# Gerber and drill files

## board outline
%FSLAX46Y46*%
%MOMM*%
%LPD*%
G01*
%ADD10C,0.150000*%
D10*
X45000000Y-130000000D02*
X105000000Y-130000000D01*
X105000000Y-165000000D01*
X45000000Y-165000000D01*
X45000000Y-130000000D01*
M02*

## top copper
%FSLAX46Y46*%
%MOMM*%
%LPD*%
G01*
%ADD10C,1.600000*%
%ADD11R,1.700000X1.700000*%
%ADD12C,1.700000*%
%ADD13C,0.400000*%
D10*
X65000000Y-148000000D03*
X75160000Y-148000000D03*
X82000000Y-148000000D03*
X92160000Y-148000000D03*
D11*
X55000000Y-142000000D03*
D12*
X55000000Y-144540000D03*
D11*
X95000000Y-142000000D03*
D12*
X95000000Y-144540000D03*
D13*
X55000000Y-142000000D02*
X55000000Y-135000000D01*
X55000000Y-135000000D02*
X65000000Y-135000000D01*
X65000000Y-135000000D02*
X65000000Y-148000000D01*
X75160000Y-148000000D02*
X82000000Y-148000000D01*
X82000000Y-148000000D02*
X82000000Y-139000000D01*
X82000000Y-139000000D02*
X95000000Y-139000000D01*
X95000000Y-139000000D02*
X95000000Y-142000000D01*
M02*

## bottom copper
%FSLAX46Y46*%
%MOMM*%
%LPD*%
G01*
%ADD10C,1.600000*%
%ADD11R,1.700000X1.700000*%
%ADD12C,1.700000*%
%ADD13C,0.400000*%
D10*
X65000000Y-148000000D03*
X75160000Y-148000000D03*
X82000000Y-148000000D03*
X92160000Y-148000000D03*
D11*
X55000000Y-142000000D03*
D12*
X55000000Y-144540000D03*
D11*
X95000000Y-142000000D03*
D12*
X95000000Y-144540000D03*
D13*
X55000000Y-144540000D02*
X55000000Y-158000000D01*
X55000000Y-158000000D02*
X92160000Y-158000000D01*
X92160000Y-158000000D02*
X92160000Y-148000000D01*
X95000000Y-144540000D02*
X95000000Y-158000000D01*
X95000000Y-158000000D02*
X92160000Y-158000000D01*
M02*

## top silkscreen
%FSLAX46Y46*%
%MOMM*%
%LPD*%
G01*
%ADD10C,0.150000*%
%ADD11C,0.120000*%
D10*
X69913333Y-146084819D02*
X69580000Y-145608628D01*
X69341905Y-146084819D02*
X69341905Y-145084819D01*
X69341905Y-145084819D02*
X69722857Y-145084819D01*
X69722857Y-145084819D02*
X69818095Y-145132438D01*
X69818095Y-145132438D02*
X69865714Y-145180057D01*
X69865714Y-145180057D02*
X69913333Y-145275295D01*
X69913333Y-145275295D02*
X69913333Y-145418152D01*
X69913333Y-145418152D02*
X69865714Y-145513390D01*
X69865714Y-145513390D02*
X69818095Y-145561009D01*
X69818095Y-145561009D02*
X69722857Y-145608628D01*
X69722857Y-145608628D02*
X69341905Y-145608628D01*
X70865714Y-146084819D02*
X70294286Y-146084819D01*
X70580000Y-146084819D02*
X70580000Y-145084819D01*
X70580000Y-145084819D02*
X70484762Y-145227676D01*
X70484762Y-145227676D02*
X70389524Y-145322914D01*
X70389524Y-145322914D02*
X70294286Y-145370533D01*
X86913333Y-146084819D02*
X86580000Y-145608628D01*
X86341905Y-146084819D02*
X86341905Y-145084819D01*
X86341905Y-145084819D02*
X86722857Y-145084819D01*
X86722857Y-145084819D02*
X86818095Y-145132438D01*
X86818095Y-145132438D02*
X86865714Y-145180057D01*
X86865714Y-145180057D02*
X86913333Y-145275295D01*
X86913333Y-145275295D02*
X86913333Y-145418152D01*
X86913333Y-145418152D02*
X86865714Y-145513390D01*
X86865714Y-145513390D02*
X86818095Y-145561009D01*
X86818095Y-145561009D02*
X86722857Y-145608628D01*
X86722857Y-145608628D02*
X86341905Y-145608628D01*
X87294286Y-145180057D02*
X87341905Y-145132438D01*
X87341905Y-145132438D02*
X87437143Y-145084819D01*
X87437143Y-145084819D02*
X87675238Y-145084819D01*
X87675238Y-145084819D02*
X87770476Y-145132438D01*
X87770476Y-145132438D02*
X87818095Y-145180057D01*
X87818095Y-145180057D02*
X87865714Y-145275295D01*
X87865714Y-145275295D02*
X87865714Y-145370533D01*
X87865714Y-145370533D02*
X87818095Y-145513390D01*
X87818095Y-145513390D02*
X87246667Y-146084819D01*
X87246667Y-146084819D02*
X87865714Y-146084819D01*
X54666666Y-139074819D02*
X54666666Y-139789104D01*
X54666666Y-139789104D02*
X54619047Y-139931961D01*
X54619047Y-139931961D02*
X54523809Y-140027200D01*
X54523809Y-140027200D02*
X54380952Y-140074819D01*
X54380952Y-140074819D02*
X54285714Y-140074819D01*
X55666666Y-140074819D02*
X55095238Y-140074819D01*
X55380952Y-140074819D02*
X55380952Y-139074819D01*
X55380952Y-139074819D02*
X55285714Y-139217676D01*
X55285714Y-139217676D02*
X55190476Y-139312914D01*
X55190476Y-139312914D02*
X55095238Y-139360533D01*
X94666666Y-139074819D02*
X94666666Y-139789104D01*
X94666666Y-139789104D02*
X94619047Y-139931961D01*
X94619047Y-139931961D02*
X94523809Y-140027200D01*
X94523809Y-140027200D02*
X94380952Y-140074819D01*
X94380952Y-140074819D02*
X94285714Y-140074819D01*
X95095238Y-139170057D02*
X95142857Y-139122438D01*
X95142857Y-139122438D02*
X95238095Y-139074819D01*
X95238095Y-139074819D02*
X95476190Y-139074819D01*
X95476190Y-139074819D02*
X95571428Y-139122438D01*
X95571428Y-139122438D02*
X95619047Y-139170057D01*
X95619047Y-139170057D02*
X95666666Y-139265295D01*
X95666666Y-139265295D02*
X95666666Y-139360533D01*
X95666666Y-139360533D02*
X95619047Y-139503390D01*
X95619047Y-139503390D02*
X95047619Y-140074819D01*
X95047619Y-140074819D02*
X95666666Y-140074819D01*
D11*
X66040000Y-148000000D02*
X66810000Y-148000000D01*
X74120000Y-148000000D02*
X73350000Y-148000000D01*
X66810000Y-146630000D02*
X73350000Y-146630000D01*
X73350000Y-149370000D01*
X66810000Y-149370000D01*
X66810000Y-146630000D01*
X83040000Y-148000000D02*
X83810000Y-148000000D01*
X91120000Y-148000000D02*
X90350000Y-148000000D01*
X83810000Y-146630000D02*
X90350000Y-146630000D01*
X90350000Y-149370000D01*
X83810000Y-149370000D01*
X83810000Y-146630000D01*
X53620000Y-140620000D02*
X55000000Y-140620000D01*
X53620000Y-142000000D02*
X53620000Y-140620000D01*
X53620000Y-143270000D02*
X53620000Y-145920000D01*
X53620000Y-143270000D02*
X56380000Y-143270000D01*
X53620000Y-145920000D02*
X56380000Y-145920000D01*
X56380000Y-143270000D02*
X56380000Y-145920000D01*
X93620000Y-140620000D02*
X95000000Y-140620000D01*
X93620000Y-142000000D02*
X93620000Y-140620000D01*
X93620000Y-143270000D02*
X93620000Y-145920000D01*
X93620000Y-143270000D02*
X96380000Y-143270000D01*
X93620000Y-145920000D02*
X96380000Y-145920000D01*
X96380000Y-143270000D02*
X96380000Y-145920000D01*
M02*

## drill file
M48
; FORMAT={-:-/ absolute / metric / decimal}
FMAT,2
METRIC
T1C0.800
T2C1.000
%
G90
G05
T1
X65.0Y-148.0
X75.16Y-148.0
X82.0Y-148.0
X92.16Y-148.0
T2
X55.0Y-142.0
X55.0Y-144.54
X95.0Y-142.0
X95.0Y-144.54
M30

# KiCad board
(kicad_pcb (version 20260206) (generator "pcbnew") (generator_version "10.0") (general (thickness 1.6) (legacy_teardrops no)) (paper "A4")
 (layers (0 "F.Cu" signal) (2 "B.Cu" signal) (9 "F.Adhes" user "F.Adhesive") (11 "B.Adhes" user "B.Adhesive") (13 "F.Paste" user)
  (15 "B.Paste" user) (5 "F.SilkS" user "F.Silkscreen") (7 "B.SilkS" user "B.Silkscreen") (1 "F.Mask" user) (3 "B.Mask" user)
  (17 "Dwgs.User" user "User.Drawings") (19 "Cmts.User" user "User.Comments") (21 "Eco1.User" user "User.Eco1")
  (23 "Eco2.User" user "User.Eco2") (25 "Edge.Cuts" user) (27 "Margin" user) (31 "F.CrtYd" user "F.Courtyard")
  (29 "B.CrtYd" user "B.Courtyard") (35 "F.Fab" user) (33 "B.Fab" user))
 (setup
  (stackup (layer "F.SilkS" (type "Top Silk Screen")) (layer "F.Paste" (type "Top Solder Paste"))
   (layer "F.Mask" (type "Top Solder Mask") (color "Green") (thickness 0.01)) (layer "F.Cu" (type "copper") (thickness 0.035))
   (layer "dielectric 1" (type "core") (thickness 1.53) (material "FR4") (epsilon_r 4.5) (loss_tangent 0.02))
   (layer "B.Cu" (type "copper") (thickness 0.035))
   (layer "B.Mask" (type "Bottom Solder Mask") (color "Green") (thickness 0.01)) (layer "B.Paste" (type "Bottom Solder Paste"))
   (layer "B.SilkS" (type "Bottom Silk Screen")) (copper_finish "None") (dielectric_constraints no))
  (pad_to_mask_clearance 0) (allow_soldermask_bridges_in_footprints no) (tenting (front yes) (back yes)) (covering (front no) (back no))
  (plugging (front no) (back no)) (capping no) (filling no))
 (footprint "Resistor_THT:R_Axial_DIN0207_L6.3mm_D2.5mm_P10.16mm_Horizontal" (layer "F.Cu") (at 65 148)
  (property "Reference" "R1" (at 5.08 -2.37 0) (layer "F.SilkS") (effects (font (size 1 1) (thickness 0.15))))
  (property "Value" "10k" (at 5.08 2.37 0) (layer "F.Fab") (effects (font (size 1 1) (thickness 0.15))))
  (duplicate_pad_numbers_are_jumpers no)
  (fp_line (start 1.04 0) (end 1.81 0) (stroke (width 0.12) (type solid)) (layer "F.SilkS"))
  (fp_line (start 9.12 0) (end 8.35 0) (stroke (width 0.12) (type solid)) (layer "F.SilkS"))
  (fp_rect (start 1.81 -1.37) (end 8.35 1.37) (stroke (width 0.12) (type solid)) (fill no) (layer "F.SilkS"))
  (pad "1" thru_hole circle (at 0 0) (size 1.6 1.6) (drill 0.8) (layers "*.Cu" "*.Mask") (remove_unused_layers no) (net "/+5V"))
  (pad "2" thru_hole circle (at 10.16 0) (size 1.6 1.6) (drill 0.8) (layers "*.Cu" "*.Mask") (remove_unused_layers no) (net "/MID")))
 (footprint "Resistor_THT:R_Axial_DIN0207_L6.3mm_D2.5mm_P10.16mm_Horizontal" (layer "F.Cu") (at 82 148 0)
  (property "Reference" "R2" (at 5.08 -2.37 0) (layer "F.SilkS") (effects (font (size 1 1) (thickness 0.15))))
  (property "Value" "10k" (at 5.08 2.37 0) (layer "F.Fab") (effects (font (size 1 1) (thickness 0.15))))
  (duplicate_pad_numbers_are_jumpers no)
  (fp_line (start 1.04 0) (end 1.81 0) (stroke (width 0.12) (type solid)) (layer "F.SilkS"))
  (fp_line (start 9.12 0) (end 8.35 0) (stroke (width 0.12) (type solid)) (layer "F.SilkS"))
  (fp_rect (start 1.81 -1.37) (end 8.35 1.37) (stroke (width 0.12) (type solid)) (fill no) (layer "F.SilkS"))
  (pad "1" thru_hole circle (at 0 0) (size 1.6 1.6) (drill 0.8) (layers "*.Cu" "*.Mask") (remove_unused_layers no) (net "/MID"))
  (pad "2" thru_hole circle (at 10.16 0) (size 1.6 1.6) (drill 0.8) (layers "*.Cu" "*.Mask") (remove_unused_layers no) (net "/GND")))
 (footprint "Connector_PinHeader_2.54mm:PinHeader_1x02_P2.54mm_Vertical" (layer "F.Cu") (at 55 142)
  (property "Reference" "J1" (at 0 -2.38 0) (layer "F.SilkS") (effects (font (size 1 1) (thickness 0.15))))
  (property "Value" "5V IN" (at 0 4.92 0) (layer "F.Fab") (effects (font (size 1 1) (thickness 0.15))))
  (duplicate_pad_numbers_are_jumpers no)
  (fp_line (start -1.38 -1.38) (end 0 -1.38) (stroke (width 0.12) (type solid)) (layer "F.SilkS"))
  (fp_line (start -1.38 0) (end -1.38 -1.38) (stroke (width 0.12) (type solid)) (layer "F.SilkS"))
  (fp_line (start -1.38 1.27) (end -1.38 3.92) (stroke (width 0.12) (type solid)) (layer "F.SilkS"))
  (fp_line (start -1.38 1.27) (end 1.38 1.27) (stroke (width 0.12) (type solid)) (layer "F.SilkS"))
  (fp_line (start -1.38 3.92) (end 1.38 3.92) (stroke (width 0.12) (type solid)) (layer "F.SilkS"))
  (fp_line (start 1.38 1.27) (end 1.38 3.92) (stroke (width 0.12) (type solid)) (layer "F.SilkS"))
  (pad "1" thru_hole rect (at 0 0) (size 1.7 1.7) (drill 1) (layers "*.Cu" "*.Mask") (remove_unused_layers no) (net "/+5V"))
  (pad "2" thru_hole circle (at 0 2.54) (size 1.7 1.7) (drill 1) (layers "*.Cu" "*.Mask") (remove_unused_layers no) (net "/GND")))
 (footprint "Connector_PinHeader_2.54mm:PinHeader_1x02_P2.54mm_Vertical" (layer "F.Cu") (at 95 142)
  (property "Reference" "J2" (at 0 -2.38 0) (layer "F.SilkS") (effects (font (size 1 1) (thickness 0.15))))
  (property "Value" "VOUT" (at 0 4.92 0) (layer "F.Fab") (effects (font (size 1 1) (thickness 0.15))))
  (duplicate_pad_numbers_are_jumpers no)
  (fp_line (start -1.38 -1.38) (end 0 -1.38) (stroke (width 0.12) (type solid)) (layer "F.SilkS"))
  (fp_line (start -1.38 0) (end -1.38 -1.38) (stroke (width 0.12) (type solid)) (layer "F.SilkS"))
  (fp_line (start -1.38 1.27) (end -1.38 3.92) (stroke (width 0.12) (type solid)) (layer "F.SilkS"))
  (fp_line (start -1.38 1.27) (end 1.38 1.27) (stroke (width 0.12) (type solid)) (layer "F.SilkS"))
  (fp_line (start -1.38 3.92) (end 1.38 3.92) (stroke (width 0.12) (type solid)) (layer "F.SilkS"))
  (fp_line (start 1.38 1.27) (end 1.38 3.92) (stroke (width 0.12) (type solid)) (layer "F.SilkS"))
  (pad "1" thru_hole rect (at 0 0) (size 1.7 1.7) (drill 1) (layers "*.Cu" "*.Mask") (remove_unused_layers no) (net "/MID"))
  (pad "2" thru_hole circle (at 0 2.54) (size 1.7 1.7) (drill 1) (layers "*.Cu" "*.Mask") (remove_unused_layers no) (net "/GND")))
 (gr_rect (start 45 130) (end 105 165) (stroke (width 0.15) (type solid)) (fill no) (layer "Edge.Cuts"))
 (segment (start 55 142) (end 55 135) (width 0.4) (layer "F.Cu") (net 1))
 (segment (start 55 135) (end 65 135) (width 0.4) (layer "F.Cu") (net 1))
 (segment (start 65 135) (end 65 148) (width 0.4) (layer "F.Cu") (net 1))
 (segment (start 75.16 148) (end 82 148) (width 0.4) (layer "F.Cu") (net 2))
 (segment (start 82 148) (end 82 139) (width 0.4) (layer "F.Cu") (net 2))
 (segment (start 82 139) (end 95 139) (width 0.4) (layer "F.Cu") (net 2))
 (segment (start 95 139) (end 95 142) (width 0.4) (layer "F.Cu") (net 2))
 (segment (start 55 144.54) (end 55 158) (width 0.4) (layer "B.Cu") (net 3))
 (segment (start 55 158) (end 92.16 158) (width 0.4) (layer "B.Cu") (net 3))
 (segment (start 92.16 158) (end 92.16 148) (width 0.4) (layer "B.Cu") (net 3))
 (segment (start 95 144.54) (end 95 158) (width 0.4) (layer "B.Cu") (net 3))
 (segment (start 95 158) (end 92.16 158) (width 0.4) (layer "B.Cu") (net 3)))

